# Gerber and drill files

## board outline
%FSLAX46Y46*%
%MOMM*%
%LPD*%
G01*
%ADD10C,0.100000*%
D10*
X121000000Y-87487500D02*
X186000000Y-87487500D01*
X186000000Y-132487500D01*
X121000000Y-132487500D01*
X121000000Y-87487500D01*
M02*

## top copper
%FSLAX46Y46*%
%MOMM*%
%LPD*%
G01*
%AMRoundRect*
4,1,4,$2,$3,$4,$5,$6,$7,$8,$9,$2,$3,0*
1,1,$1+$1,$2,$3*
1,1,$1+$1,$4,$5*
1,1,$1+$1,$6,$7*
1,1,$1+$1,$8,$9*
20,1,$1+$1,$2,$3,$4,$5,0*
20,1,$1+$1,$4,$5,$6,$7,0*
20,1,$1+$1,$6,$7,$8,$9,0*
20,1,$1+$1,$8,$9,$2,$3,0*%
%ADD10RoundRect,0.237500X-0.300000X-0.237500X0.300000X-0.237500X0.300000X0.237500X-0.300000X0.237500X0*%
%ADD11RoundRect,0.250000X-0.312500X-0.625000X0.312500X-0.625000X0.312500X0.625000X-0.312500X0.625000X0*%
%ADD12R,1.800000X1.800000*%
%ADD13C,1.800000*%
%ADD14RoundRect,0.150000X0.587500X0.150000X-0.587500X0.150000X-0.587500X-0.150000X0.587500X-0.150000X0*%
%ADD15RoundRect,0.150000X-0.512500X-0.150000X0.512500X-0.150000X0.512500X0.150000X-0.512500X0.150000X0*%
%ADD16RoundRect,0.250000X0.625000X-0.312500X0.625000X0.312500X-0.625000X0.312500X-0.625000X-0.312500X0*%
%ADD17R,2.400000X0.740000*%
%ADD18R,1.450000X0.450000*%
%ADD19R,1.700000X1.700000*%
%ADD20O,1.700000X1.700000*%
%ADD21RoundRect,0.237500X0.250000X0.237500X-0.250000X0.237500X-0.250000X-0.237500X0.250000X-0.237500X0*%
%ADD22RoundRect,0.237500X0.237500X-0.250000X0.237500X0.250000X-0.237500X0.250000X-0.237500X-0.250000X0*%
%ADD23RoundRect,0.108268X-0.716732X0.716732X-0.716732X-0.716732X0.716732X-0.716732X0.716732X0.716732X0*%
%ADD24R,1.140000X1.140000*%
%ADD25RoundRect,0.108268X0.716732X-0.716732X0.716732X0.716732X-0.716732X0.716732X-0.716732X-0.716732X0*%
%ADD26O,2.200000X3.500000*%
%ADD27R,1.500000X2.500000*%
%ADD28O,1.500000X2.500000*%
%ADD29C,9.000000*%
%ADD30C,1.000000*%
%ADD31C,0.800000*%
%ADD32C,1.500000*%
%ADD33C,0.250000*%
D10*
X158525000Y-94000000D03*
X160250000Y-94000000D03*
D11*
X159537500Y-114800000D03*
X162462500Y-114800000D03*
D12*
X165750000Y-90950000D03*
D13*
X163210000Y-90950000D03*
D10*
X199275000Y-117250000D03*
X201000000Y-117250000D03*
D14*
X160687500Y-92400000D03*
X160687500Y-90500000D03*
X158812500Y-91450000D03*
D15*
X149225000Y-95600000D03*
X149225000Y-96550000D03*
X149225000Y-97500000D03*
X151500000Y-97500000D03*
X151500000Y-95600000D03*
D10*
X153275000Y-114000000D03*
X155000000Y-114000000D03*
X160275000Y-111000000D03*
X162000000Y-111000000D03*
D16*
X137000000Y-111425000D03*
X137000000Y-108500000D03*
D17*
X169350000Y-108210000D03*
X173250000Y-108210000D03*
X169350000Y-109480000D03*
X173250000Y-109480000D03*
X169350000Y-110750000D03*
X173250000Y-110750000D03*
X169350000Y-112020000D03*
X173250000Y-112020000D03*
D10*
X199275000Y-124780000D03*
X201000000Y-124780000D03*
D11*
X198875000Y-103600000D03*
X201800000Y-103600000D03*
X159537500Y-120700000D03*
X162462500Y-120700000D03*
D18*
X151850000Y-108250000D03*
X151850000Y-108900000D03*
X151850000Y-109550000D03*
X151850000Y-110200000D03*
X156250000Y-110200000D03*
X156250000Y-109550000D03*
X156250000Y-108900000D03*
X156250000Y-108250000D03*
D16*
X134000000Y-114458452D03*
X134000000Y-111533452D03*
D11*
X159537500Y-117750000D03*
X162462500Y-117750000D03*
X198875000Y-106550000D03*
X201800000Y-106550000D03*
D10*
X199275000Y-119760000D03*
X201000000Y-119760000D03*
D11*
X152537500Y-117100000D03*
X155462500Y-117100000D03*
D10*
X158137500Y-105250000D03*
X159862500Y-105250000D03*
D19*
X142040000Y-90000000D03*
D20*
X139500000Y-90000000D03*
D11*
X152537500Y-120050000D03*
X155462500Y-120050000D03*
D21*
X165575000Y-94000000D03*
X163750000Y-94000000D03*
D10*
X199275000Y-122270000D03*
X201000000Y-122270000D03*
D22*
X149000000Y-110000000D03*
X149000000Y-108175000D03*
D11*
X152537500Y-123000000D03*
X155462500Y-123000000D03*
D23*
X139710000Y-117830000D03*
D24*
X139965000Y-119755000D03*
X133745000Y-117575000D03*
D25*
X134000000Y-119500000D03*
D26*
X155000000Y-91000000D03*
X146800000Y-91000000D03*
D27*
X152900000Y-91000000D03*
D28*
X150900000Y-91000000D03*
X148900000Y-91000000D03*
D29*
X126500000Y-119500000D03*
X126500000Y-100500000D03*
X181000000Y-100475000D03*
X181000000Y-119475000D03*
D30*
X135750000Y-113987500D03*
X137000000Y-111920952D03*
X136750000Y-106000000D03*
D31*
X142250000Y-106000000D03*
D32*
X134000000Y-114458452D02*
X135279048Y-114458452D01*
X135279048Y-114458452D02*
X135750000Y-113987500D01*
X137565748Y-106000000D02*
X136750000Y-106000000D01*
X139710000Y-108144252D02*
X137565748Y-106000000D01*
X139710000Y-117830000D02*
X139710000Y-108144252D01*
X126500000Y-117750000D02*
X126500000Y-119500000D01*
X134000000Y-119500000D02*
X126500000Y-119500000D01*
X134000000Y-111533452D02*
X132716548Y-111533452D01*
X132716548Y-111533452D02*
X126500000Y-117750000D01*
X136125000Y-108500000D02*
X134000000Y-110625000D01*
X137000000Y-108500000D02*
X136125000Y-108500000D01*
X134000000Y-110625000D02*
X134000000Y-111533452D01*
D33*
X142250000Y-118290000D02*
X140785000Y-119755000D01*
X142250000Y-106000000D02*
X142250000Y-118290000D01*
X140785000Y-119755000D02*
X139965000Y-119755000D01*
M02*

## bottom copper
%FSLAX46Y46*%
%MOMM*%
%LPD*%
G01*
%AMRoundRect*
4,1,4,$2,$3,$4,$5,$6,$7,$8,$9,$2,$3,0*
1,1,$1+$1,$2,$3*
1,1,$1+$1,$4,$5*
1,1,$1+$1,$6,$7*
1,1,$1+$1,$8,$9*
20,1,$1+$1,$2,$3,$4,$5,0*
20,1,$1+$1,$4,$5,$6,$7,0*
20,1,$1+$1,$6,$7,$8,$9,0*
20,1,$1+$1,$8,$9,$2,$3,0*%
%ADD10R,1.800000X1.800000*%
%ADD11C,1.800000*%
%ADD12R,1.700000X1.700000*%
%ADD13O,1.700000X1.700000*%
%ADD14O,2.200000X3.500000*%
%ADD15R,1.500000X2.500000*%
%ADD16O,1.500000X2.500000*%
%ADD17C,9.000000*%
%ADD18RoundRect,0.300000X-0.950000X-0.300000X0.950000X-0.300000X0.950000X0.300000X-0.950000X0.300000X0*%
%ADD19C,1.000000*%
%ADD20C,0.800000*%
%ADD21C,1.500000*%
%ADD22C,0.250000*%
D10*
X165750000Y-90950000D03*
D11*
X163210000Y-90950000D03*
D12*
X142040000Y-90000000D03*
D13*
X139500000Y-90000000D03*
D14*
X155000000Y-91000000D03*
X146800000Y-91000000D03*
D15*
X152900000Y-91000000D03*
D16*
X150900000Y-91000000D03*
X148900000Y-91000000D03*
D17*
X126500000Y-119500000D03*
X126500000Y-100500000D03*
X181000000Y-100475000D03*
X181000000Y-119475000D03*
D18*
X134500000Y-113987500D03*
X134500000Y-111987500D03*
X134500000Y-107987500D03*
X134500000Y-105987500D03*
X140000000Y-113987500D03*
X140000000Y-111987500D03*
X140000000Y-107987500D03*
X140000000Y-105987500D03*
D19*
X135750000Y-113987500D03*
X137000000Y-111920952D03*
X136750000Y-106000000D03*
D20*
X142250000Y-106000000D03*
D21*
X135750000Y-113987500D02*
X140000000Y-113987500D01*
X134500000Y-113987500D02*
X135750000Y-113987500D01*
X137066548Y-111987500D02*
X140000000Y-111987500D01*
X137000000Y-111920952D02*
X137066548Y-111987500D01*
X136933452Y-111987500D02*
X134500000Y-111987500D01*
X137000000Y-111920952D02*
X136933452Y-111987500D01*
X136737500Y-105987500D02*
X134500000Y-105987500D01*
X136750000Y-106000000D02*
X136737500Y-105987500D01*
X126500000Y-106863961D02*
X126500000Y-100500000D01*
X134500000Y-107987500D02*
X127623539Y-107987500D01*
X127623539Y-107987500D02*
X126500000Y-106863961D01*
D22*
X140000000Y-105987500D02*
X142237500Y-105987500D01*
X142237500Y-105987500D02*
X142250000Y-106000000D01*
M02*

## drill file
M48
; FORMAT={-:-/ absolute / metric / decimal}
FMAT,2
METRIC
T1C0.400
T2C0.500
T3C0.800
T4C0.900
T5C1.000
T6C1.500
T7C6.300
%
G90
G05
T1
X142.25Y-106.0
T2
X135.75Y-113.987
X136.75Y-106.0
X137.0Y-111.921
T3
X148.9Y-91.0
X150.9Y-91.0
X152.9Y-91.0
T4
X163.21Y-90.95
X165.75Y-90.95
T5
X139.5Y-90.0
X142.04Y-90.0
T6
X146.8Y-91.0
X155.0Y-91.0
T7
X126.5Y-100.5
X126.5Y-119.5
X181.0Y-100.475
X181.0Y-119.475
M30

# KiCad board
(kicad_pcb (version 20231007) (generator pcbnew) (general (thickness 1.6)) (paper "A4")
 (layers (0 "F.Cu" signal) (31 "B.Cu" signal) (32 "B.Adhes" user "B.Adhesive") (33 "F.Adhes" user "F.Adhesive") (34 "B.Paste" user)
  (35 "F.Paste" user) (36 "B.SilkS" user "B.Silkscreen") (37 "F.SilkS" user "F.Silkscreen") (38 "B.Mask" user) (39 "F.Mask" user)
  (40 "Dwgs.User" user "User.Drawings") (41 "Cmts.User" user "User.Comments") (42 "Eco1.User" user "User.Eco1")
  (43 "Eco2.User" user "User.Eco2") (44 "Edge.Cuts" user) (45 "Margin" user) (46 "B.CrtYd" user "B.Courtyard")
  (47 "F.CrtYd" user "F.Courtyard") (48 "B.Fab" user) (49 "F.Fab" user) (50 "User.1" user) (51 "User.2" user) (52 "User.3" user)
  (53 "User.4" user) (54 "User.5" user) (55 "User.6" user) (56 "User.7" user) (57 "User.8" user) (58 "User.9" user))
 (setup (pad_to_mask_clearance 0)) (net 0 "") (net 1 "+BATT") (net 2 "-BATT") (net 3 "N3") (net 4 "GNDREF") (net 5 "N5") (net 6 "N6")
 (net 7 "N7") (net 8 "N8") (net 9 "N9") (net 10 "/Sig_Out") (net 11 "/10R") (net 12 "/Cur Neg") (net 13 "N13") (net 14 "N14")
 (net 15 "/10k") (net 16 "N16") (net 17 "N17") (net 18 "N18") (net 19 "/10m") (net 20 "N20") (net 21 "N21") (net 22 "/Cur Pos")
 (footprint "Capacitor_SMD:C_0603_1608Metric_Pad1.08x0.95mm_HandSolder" (layer "F.Cu") (at 159.3875 94)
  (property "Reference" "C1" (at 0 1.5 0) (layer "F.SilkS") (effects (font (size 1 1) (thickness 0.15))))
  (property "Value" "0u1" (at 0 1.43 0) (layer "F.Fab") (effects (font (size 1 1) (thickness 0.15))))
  (pad "1" smd roundrect (at -0.8625 0) (size 1.075 0.95) (layers "F.Cu" "F.Paste" "F.Mask") (roundrect_rratio 0.25) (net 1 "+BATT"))
  (pad "2" smd roundrect (at 0.8625 0) (size 1.075 0.95) (layers "F.Cu" "F.Paste" "F.Mask") (roundrect_rratio 0.25) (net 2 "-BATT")))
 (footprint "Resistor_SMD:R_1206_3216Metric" (layer "F.Cu") (at 161 114.8)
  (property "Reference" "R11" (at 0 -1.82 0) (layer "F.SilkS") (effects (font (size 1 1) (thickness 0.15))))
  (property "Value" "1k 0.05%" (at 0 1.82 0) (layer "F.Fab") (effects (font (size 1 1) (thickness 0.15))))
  (pad "1" smd roundrect (at -1.4625 0) (size 1.125 1.75) (layers "F.Cu" "F.Paste" "F.Mask") (roundrect_rratio 0.222222) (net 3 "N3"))
  (pad "2" smd roundrect (at 1.4625 0) (size 1.125 1.75) (layers "F.Cu" "F.Paste" "F.Mask") (roundrect_rratio 0.222222) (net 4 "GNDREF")))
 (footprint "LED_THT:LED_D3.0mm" (layer "F.Cu") (at 165.75 90.95 180)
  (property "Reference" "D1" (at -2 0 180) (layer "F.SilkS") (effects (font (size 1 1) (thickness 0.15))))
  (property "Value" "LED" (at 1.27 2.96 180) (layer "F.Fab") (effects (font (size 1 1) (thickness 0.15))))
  (pad "1" thru_hole rect (at 0 0 180) (size 1.8 1.8) (drill 0.9) (layers "*.Cu" "*.Mask") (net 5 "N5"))
  (pad "2" thru_hole circle (at 2.54 0 180) (size 1.8 1.8) (drill 0.9) (layers "*.Cu" "*.Mask") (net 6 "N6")))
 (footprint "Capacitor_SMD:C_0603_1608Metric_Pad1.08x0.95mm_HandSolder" (layer "F.Cu") (at 200.1375 117.25)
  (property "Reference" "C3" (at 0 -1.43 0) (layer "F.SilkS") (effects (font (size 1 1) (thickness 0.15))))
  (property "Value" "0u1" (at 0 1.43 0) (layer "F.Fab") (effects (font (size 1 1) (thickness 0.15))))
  (pad "1" smd roundrect (at -0.8625 0) (size 1.075 0.95) (layers "F.Cu" "F.Paste" "F.Mask") (roundrect_rratio 0.25) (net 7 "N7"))
  (pad "2" smd roundrect (at 0.8625 0) (size 1.075 0.95) (layers "F.Cu" "F.Paste" "F.Mask") (roundrect_rratio 0.25) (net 2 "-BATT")))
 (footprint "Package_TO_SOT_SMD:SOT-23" (layer "F.Cu") (at 159.75 91.45 180)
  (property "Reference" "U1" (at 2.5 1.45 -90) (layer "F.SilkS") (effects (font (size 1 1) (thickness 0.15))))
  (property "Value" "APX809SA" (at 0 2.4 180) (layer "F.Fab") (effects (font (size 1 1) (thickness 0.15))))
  (pad "1" smd roundrect (at -0.9375 -0.95 180) (size 1.475 0.6) (layers "F.Cu" "F.Paste" "F.Mask") (roundrect_rratio 0.25) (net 2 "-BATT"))
  (pad "2" smd roundrect (at -0.9375 0.95 180) (size 1.475 0.6) (layers "F.Cu" "F.Paste" "F.Mask") (roundrect_rratio 0.25) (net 6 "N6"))
  (pad "3" smd roundrect (at 0.9375 0 180) (size 1.475 0.6) (layers "F.Cu" "F.Paste" "F.Mask") (roundrect_rratio 0.25) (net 1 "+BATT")))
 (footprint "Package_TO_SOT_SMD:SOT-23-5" (layer "F.Cu") (at 150.3625 96.55)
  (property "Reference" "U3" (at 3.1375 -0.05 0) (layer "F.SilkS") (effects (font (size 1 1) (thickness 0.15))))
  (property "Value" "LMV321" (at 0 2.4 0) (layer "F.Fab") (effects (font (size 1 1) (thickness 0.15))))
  (pad "1" smd roundrect (at -1.1375 -0.95) (size 1.325 0.6) (layers "F.Cu" "F.Paste" "F.Mask") (roundrect_rratio 0.25) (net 7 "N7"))
  (pad "2" smd roundrect (at -1.1375 0) (size 1.325 0.6) (layers "F.Cu" "F.Paste" "F.Mask") (roundrect_rratio 0.25) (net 2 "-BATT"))
  (pad "3" smd roundrect (at -1.1375 0.95) (size 1.325 0.6) (layers "F.Cu" "F.Paste" "F.Mask") (roundrect_rratio 0.25) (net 4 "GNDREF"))
  (pad "4" smd roundrect (at 1.1375 0.95) (size 1.325 0.6) (layers "F.Cu" "F.Paste" "F.Mask") (roundrect_rratio 0.25) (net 4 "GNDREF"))
  (pad "5" smd roundrect (at 1.1375 -0.95) (size 1.325 0.6) (layers "F.Cu" "F.Paste" "F.Mask") (roundrect_rratio 0.25) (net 1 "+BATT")))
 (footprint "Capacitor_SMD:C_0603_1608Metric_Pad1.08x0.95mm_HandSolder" (layer "F.Cu") (at 154.1375 114)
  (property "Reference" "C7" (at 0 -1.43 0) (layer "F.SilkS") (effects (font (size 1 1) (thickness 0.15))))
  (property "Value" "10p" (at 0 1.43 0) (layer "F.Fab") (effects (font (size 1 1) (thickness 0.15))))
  (pad "1" smd roundrect (at -0.8625 0) (size 1.075 0.95) (layers "F.Cu" "F.Paste" "F.Mask") (roundrect_rratio 0.25) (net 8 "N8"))
  (pad "2" smd roundrect (at 0.8625 0) (size 1.075 0.95) (layers "F.Cu" "F.Paste" "F.Mask") (roundrect_rratio 0.25) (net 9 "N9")))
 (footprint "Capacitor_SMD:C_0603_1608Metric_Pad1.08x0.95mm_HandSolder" (layer "F.Cu") (at 161.1375 111)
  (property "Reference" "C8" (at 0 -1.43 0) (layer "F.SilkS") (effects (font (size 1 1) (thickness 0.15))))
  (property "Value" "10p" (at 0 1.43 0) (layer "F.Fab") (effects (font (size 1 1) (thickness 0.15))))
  (pad "1" smd roundrect (at -0.8625 0) (size 1.075 0.95) (layers "F.Cu" "F.Paste" "F.Mask") (roundrect_rratio 0.25) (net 3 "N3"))
  (pad "2" smd roundrect (at 0.8625 0) (size 1.075 0.95) (layers "F.Cu" "F.Paste" "F.Mask") (roundrect_rratio 0.25) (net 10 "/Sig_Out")))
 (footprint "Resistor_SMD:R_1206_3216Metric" (layer "F.Cu") (at 137 109.9625 90)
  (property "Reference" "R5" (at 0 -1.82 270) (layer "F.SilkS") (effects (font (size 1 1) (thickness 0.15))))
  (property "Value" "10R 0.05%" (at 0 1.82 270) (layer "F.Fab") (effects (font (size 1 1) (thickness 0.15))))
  (pad "1" smd roundrect (at -1.4625 0 90) (size 1.125 1.75) (layers "F.Cu" "F.Paste" "F.Mask") (roundrect_rratio 0.222222) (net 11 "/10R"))
  (pad "2" smd roundrect (at 1.4625 0 90) (size 1.125 1.75) (layers "F.Cu" "F.Paste" "F.Mask") (roundrect_rratio 0.222222)
   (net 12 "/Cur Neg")))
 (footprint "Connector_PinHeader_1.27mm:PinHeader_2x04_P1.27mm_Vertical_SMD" (layer "F.Cu") (at 171.3 110.115)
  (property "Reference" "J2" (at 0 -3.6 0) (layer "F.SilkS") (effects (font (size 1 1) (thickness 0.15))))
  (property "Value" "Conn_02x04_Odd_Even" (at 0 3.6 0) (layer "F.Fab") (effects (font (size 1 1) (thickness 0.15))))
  (pad "1" smd rect (at -1.95 -1.905) (size 2.4 0.74) (layers "F.Cu" "F.Paste" "F.Mask") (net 1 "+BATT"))
  (pad "2" smd rect (at 1.95 -1.905) (size 2.4 0.74) (layers "F.Cu" "F.Paste" "F.Mask") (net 1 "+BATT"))
  (pad "3" smd rect (at -1.95 -0.635) (size 2.4 0.74) (layers "F.Cu" "F.Paste" "F.Mask") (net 10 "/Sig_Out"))
  (pad "4" smd rect (at 1.95 -0.635) (size 2.4 0.74) (layers "F.Cu" "F.Paste" "F.Mask") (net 10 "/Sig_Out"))
  (pad "5" smd rect (at -1.95 0.635) (size 2.4 0.74) (layers "F.Cu" "F.Paste" "F.Mask") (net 4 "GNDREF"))
  (pad "6" smd rect (at 1.95 0.635) (size 2.4 0.74) (layers "F.Cu" "F.Paste" "F.Mask") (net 4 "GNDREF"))
  (pad "7" smd rect (at -1.95 1.905) (size 2.4 0.74) (layers "F.Cu" "F.Paste" "F.Mask") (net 2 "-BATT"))
  (pad "8" smd rect (at 1.95 1.905) (size 2.4 0.74) (layers "F.Cu" "F.Paste" "F.Mask") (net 2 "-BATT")))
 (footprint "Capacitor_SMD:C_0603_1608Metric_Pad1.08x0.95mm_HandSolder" (layer "F.Cu") (at 200.1375 124.78)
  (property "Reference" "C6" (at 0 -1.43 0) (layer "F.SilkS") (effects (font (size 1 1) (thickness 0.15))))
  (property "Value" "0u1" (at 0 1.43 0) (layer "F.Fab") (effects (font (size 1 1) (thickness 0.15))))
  (pad "1" smd roundrect (at -0.8625 0) (size 1.075 0.95) (layers "F.Cu" "F.Paste" "F.Mask") (roundrect_rratio 0.25) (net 4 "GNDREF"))
  (pad "2" smd roundrect (at 0.8625 0) (size 1.075 0.95) (layers "F.Cu" "F.Paste" "F.Mask") (roundrect_rratio 0.25) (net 2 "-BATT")))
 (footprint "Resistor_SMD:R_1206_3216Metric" (layer "F.Cu") (at 200.3375 103.6)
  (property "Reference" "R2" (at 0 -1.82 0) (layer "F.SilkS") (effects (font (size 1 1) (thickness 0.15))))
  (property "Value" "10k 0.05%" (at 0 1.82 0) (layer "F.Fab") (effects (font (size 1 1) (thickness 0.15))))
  (pad "1" smd roundrect (at -1.4625 0) (size 1.125 1.75) (layers "F.Cu" "F.Paste" "F.Mask") (roundrect_rratio 0.222222) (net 1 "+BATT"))
  (pad "2" smd roundrect (at 1.4625 0) (size 1.125 1.75) (layers "F.Cu" "F.Paste" "F.Mask") (roundrect_rratio 0.222222) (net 7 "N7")))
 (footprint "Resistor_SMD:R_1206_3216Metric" (layer "F.Cu") (at 161 120.7)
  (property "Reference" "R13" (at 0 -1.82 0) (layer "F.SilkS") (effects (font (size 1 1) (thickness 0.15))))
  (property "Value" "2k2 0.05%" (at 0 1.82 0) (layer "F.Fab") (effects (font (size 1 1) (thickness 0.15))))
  (pad "1" smd roundrect (at -1.4625 0) (size 1.125 1.75) (layers "F.Cu" "F.Paste" "F.Mask") (roundrect_rratio 0.222222) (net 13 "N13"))
  (pad "2" smd roundrect (at 1.4625 0) (size 1.125 1.75) (layers "F.Cu" "F.Paste" "F.Mask") (roundrect_rratio 0.222222) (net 10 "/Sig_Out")))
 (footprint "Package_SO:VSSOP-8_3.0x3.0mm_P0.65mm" (layer "F.Cu") (at 154.05 109.225)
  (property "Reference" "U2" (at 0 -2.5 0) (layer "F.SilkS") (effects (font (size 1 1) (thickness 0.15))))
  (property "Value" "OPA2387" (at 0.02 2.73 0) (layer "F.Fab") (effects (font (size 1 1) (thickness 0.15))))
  (pad "1" smd rect (at -2.2 -0.975 270) (size 0.45 1.45) (layers "F.Cu" "F.Paste" "F.Mask") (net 9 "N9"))
  (pad "2" smd rect (at -2.2 -0.325 270) (size 0.45 1.45) (layers "F.Cu" "F.Paste" "F.Mask") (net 8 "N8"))
  (pad "3" smd rect (at -2.2 0.325 270) (size 0.45 1.45) (layers "F.Cu" "F.Paste" "F.Mask") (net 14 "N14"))
  (pad "4" smd rect (at -2.2 0.975 270) (size 0.45 1.45) (layers "F.Cu" "F.Paste" "F.Mask") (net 2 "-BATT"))
  (pad "5" smd rect (at 2.2 0.975 270) (size 0.45 1.45) (layers "F.Cu" "F.Paste" "F.Mask") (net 9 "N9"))
  (pad "6" smd rect (at 2.2 0.325 270) (size 0.45 1.45) (layers "F.Cu" "F.Paste" "F.Mask") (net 3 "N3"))
  (pad "7" smd rect (at 2.2 -0.325 270) (size 0.45 1.45) (layers "F.Cu" "F.Paste" "F.Mask") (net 10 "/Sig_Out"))
  (pad "8" smd rect (at 2.2 -0.975 270) (size 0.45 1.45) (layers "F.Cu" "F.Paste" "F.Mask") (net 1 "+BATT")))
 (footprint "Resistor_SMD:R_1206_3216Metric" (layer "F.Cu") (at 134 112.995952 90)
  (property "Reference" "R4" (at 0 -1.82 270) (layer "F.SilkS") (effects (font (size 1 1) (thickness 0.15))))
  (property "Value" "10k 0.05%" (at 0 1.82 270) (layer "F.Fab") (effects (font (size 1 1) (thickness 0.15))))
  (pad "1" smd roundrect (at -1.4625 0 90) (size 1.125 1.75) (layers "F.Cu" "F.Paste" "F.Mask") (roundrect_rratio 0.222222) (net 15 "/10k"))
  (pad "2" smd roundrect (at 1.4625 0 90) (size 1.125 1.75) (layers "F.Cu" "F.Paste" "F.Mask") (roundrect_rratio 0.222222)
   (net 12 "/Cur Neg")))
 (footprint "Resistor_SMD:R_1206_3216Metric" (layer "F.Cu") (at 161 117.75)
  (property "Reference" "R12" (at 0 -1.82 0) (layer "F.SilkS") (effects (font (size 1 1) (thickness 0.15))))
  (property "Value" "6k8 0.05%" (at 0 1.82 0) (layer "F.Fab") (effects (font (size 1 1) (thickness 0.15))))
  (pad "1" smd roundrect (at -1.4625 0) (size 1.125 1.75) (layers "F.Cu" "F.Paste" "F.Mask") (roundrect_rratio 0.222222) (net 3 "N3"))
  (pad "2" smd roundrect (at 1.4625 0) (size 1.125 1.75) (layers "F.Cu" "F.Paste" "F.Mask") (roundrect_rratio 0.222222) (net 13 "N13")))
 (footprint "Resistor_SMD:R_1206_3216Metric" (layer "F.Cu") (at 200.3375 106.55)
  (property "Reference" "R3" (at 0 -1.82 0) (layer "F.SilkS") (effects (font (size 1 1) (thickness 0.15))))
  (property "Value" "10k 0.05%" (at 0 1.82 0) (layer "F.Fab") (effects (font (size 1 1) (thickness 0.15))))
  (pad "1" smd roundrect (at -1.4625 0) (size 1.125 1.75) (layers "F.Cu" "F.Paste" "F.Mask") (roundrect_rratio 0.222222) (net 7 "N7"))
  (pad "2" smd roundrect (at 1.4625 0) (size 1.125 1.75) (layers "F.Cu" "F.Paste" "F.Mask") (roundrect_rratio 0.222222) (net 2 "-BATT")))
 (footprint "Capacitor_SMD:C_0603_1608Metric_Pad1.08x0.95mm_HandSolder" (layer "F.Cu") (at 200.1375 119.76)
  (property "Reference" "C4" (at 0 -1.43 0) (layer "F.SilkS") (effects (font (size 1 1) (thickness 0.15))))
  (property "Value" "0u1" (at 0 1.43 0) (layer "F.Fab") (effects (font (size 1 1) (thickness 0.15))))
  (pad "1" smd roundrect (at -0.8625 0) (size 1.075 0.95) (layers "F.Cu" "F.Paste" "F.Mask") (roundrect_rratio 0.25) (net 1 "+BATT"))
  (pad "2" smd roundrect (at 0.8625 0) (size 1.075 0.95) (layers "F.Cu" "F.Paste" "F.Mask") (roundrect_rratio 0.25) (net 2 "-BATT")))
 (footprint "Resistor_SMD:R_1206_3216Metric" (layer "F.Cu") (at 154 117.1)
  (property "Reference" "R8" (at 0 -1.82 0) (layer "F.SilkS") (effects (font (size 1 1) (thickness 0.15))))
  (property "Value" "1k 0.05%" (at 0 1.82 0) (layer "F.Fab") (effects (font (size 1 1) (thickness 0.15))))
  (pad "1" smd roundrect (at -1.4625 0) (size 1.125 1.75) (layers "F.Cu" "F.Paste" "F.Mask") (roundrect_rratio 0.222222) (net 8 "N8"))
  (pad "2" smd roundrect (at 1.4625 0) (size 1.125 1.75) (layers "F.Cu" "F.Paste" "F.Mask") (roundrect_rratio 0.222222) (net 4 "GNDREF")))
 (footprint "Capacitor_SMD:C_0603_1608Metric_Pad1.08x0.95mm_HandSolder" (layer "F.Cu") (at 159 105.25)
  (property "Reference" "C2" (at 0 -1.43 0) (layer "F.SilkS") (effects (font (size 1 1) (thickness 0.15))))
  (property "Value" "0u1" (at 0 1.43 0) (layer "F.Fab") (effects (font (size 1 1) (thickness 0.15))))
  (pad "1" smd roundrect (at -0.8625 0) (size 1.075 0.95) (layers "F.Cu" "F.Paste" "F.Mask") (roundrect_rratio 0.25) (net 1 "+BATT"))
  (pad "2" smd roundrect (at 0.8625 0) (size 1.075 0.95) (layers "F.Cu" "F.Paste" "F.Mask") (roundrect_rratio 0.25) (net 2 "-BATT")))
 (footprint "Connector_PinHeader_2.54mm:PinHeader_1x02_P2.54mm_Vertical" (layer "F.Cu") (at 142.04 90 -90)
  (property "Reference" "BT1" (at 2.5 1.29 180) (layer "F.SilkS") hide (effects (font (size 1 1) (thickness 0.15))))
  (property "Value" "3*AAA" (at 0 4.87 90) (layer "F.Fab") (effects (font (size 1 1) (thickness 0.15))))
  (pad "1" thru_hole rect (at 0 0 270) (size 1.7 1.7) (drill 1) (layers "*.Cu" "*.Mask") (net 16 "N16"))
  (pad "2" thru_hole oval (at 0 2.54 270) (size 1.7 1.7) (drill 1) (layers "*.Cu" "*.Mask") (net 2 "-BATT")))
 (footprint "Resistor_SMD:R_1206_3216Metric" (layer "F.Cu") (at 154 120.05)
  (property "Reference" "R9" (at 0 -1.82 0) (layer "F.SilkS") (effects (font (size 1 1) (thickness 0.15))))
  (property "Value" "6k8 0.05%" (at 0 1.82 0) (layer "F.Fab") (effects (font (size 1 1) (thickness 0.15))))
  (pad "1" smd roundrect (at -1.4625 0) (size 1.125 1.75) (layers "F.Cu" "F.Paste" "F.Mask") (roundrect_rratio 0.222222) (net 8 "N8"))
  (pad "2" smd roundrect (at 1.4625 0) (size 1.125 1.75) (layers "F.Cu" "F.Paste" "F.Mask") (roundrect_rratio 0.222222) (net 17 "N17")))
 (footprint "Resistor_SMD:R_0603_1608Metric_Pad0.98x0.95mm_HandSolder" (layer "F.Cu") (at 164.6625 94 180)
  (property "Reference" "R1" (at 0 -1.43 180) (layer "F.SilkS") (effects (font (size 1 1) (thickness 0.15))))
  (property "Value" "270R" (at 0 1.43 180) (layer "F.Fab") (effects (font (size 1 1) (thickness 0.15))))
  (pad "1" smd roundrect (at -0.9125 0 180) (size 0.975 0.95) (layers "F.Cu" "F.Paste" "F.Mask") (roundrect_rratio 0.25) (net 5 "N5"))
  (pad "2" smd roundrect (at 0.9125 0 180) (size 0.975 0.95) (layers "F.Cu" "F.Paste" "F.Mask") (roundrect_rratio 0.25) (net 2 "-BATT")))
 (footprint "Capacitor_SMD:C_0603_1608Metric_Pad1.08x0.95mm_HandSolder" (layer "F.Cu") (at 200.1375 122.27)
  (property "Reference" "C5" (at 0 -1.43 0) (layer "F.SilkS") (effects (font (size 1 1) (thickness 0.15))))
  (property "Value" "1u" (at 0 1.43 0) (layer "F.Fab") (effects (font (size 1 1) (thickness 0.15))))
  (pad "1" smd roundrect (at -0.8625 0) (size 1.075 0.95) (layers "F.Cu" "F.Paste" "F.Mask") (roundrect_rratio 0.25) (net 4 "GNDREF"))
  (pad "2" smd roundrect (at 0.8625 0) (size 1.075 0.95) (layers "F.Cu" "F.Paste" "F.Mask") (roundrect_rratio 0.25) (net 2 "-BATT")))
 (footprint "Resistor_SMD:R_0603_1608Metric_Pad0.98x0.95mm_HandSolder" (layer "F.Cu") (at 149 109.0875 90)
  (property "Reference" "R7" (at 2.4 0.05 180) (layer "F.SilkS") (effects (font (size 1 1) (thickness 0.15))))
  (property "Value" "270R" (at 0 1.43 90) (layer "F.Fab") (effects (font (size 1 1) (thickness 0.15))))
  (pad "1" smd roundrect (at -0.9125 0 90) (size 0.975 0.95) (layers "F.Cu" "F.Paste" "F.Mask") (roundrect_rratio 0.25) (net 14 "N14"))
  (pad "2" smd roundrect (at 0.9125 0 90) (size 0.975 0.95) (layers "F.Cu" "F.Paste" "F.Mask") (roundrect_rratio 0.25) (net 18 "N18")))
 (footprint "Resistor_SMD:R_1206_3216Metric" (layer "F.Cu") (at 154 123)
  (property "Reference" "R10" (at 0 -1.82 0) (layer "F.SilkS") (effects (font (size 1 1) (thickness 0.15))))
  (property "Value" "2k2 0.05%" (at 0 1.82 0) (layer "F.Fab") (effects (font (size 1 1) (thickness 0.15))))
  (pad "1" smd roundrect (at -1.4625 0) (size 1.125 1.75) (layers "F.Cu" "F.Paste" "F.Mask") (roundrect_rratio 0.222222) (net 17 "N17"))
  (pad "2" smd roundrect (at 1.4625 0) (size 1.125 1.75) (layers "F.Cu" "F.Paste" "F.Mask") (roundrect_rratio 0.222222) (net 9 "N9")))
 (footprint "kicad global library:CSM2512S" (layer "F.Cu") (at 139.71 117.83 -90)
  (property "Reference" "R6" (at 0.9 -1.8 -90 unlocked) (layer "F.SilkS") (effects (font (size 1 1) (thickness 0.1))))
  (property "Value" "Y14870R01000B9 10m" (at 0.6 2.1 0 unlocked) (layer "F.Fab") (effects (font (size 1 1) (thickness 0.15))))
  (pad "1" smd roundrect (at 0 0 270) (size 1.65 1.65) (layers "F.Cu" "F.Paste" "F.Mask") (roundrect_rratio 0.0656167979) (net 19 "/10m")
   (thermal_bridge_angle 45))
  (pad "2" smd rect (at 1.925 -0.255 270) (size 1.14 1.14) (layers "F.Cu" "F.Paste" "F.Mask") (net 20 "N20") (thermal_bridge_angle 45))
  (pad "3" smd rect (at -0.255 5.965 90) (size 1.14 1.14) (layers "F.Cu" "F.Paste" "F.Mask") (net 4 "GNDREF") (thermal_bridge_angle 45))
  (pad "4" smd roundrect (at 1.67 5.71 90) (size 1.65 1.65) (layers "F.Cu" "F.Paste" "F.Mask") (roundrect_rratio 0.0656167979)
   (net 12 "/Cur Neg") (thermal_bridge_angle 45)))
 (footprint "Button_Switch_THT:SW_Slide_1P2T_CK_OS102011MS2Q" (layer "B.Cu") (at 152.9 91 180)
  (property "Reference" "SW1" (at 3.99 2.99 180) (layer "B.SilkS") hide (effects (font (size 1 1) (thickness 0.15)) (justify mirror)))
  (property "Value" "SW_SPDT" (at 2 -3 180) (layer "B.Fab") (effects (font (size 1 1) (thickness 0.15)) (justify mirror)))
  (pad "" thru_hole oval (at -2.1 0 180) (size 2.2 3.5) (drill 1.5) (layers "*.Cu" "*.Mask"))
  (pad "" thru_hole oval (at 6.1 0 180) (size 2.2 3.5) (drill 1.5) (layers "*.Cu" "*.Mask"))
  (pad "1" thru_hole rect (at 0 0 180) (size 1.5 2.5) (drill 0.8) (layers "*.Cu" "*.Mask") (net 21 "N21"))
  (pad "2" thru_hole oval (at 2 0 180) (size 1.5 2.5) (drill 0.8) (layers "*.Cu" "*.Mask") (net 16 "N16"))
  (pad "3" thru_hole oval (at 4 0 180) (size 1.5 2.5) (drill 0.8) (layers "*.Cu" "*.Mask") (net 1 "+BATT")))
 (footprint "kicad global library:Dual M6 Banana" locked (layer "B.Cu") (at 126.5 119.5 90)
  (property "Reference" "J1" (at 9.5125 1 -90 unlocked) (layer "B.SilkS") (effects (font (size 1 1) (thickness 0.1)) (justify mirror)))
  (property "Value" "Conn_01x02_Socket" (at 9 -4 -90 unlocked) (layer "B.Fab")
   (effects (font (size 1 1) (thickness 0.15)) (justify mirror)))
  (pad "1" thru_hole circle locked (at 0 0 90) (size 9 9) (drill 6.3) (layers "*.Cu" "*.Mask") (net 12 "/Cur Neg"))
  (pad "2" thru_hole circle locked (at 19 0 90) (size 9 9) (drill 6.3) (layers "*.Cu" "*.Mask") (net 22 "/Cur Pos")))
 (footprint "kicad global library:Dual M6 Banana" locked (layer "B.Cu") (at 181 100.475 -90)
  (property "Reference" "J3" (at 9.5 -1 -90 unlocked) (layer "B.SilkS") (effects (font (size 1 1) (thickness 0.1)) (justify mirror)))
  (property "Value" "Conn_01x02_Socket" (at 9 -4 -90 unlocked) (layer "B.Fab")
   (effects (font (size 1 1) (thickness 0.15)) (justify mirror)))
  (pad "1" thru_hole circle locked (at 0 0 270) (size 9 9) (drill 6.3) (layers "*.Cu" "*.Mask") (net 10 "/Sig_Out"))
  (pad "2" thru_hole circle locked (at 19 0 270) (size 9 9) (drill 6.3) (layers "*.Cu" "*.Mask") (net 4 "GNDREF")))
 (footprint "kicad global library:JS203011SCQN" (layer "B.Cu") (at 134.5 113.9875 90)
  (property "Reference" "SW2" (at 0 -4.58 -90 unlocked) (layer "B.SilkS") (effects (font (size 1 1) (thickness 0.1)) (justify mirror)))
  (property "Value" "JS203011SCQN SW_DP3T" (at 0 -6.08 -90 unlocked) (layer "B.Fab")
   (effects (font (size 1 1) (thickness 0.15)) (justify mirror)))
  (pad "1" smd roundrect (at 0 0) (size 2.5 1.2) (layers "B.Cu" "B.Paste" "B.Mask") (roundrect_rratio 0.25) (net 15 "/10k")
   (thermal_bridge_angle 45))
  (pad "2" smd roundrect (at 2 0) (size 2.5 1.2) (layers "B.Cu" "B.Paste" "B.Mask") (roundrect_rratio 0.25) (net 11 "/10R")
   (thermal_bridge_angle 45))
  (pad "3" smd roundrect (at 6 0) (size 2.5 1.2) (layers "B.Cu" "B.Paste" "B.Mask") (roundrect_rratio 0.25) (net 22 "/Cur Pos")
   (thermal_bridge_angle 45))
  (pad "4" smd roundrect (at 8 0) (size 2.5 1.2) (layers "B.Cu" "B.Paste" "B.Mask") (roundrect_rratio 0.25) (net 19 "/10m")
   (thermal_bridge_angle 45))
  (pad "5" smd roundrect (at 0 5.5) (size 2.5 1.2) (layers "B.Cu" "B.Paste" "B.Mask") (roundrect_rratio 0.25) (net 15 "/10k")
   (thermal_bridge_angle 45))
  (pad "6" smd roundrect (at 2 5.5) (size 2.5 1.2) (layers "B.Cu" "B.Paste" "B.Mask") (roundrect_rratio 0.25) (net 11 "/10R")
   (thermal_bridge_angle 45))
  (pad "7" smd roundrect (at 6 5.5) (size 2.5 1.2) (layers "B.Cu" "B.Paste" "B.Mask") (roundrect_rratio 0.25) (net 18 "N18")
   (thermal_bridge_angle 45))
  (pad "8" smd roundrect (at 8 5.5) (size 2.5 1.2) (layers "B.Cu" "B.Paste" "B.Mask") (roundrect_rratio 0.25) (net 20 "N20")
   (thermal_bridge_angle 45)))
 (gr_rect locked (start 121 87.4875) (end 186 132.4875) (stroke (width 0.1) (type default)) (fill none) (layer "Edge.Cuts"))
 (segment (start 134 114.458452) (end 135.279048 114.458452) (width 1.5) (layer "F.Cu") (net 15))
 (segment (start 135.279048 114.458452) (end 135.75 113.9875) (width 1.5) (layer "F.Cu") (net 15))
 (via (at 135.75 113.9875) (size 1) (drill 0.5) (layers "F.Cu" "B.Cu") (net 15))
 (segment (start 135.75 113.9875) (end 140 113.9875) (width 1.5) (layer "B.Cu") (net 15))
 (segment (start 134.5 113.9875) (end 135.75 113.9875) (width 1.5) (layer "B.Cu") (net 15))
 (via (at 137 111.920952) (size 1) (drill 0.5) (layers "F.Cu" "B.Cu") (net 11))
 (segment (start 137.066548 111.9875) (end 140 111.9875) (width 1.5) (layer "B.Cu") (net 11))
 (segment (start 137 111.920952) (end 137.066548 111.9875) (width 1.5) (layer "B.Cu") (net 11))
 (segment (start 136.933452 111.9875) (end 134.5 111.9875) (width 1.5) (layer "B.Cu") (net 11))
 (segment (start 137 111.920952) (end 136.933452 111.9875) (width 1.5) (layer "B.Cu") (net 11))
 (segment (start 137.565748 106) (end 136.75 106) (width 1.5) (layer "F.Cu") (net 19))
 (segment (start 139.71 108.144252) (end 137.565748 106) (width 1.5) (layer "F.Cu") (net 19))
 (segment (start 139.71 117.83) (end 139.71 108.144252) (width 1.5) (layer "F.Cu") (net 19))
 (via (at 136.75 106) (size 1) (drill 0.5) (layers "F.Cu" "B.Cu") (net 19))
 (segment (start 136.7375 105.9875) (end 134.5 105.9875) (width 1.5) (layer "B.Cu") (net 19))
 (segment (start 136.75 106) (end 136.7375 105.9875) (width 1.5) (layer "B.Cu") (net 19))
 (segment (start 126.5 117.75) (end 126.5 119.5) (width 1.5) (layer "F.Cu") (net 12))
 (segment (start 134 119.5) (end 126.5 119.5) (width 1.5) (layer "F.Cu") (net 12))
 (segment (start 134 111.533452) (end 132.716548 111.533452) (width 1.5) (layer "F.Cu") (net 12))
 (segment (start 132.716548 111.533452) (end 126.5 117.75) (width 1.5) (layer "F.Cu") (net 12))
 (segment (start 136.125 108.5) (end 134 110.625) (width 1.5) (layer "F.Cu") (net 12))
 (segment (start 137 108.5) (end 136.125 108.5) (width 1.5) (layer "F.Cu") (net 12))
 (segment (start 134 110.625) (end 134 111.533452) (width 1.5) (layer "F.Cu") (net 12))
 (segment (start 126.5 106.863961) (end 126.5 100.5) (width 1.5) (layer "B.Cu") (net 22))
 (segment (start 134.5 107.9875) (end 127.623539 107.9875) (width 1.5) (layer "B.Cu") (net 22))
 (segment (start 127.623539 107.9875) (end 126.5 106.863961) (width 1.5) (layer "B.Cu") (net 22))
 (segment (start 142.25 118.29) (end 140.785 119.755) (width 0.25) (layer "F.Cu") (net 20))
 (segment (start 142.25 106) (end 142.25 118.29) (width 0.25) (layer "F.Cu") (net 20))
 (segment (start 140.785 119.755) (end 139.965 119.755) (width 0.25) (layer "F.Cu") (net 20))
 (via (at 142.25 106) (size 0.8) (drill 0.4) (layers "F.Cu" "B.Cu") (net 20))
 (segment (start 140 105.9875) (end 142.2375 105.9875) (width 0.25) (layer "B.Cu") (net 20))
 (segment (start 142.2375 105.9875) (end 142.25 106) (width 0.25) (layer "B.Cu") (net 20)))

